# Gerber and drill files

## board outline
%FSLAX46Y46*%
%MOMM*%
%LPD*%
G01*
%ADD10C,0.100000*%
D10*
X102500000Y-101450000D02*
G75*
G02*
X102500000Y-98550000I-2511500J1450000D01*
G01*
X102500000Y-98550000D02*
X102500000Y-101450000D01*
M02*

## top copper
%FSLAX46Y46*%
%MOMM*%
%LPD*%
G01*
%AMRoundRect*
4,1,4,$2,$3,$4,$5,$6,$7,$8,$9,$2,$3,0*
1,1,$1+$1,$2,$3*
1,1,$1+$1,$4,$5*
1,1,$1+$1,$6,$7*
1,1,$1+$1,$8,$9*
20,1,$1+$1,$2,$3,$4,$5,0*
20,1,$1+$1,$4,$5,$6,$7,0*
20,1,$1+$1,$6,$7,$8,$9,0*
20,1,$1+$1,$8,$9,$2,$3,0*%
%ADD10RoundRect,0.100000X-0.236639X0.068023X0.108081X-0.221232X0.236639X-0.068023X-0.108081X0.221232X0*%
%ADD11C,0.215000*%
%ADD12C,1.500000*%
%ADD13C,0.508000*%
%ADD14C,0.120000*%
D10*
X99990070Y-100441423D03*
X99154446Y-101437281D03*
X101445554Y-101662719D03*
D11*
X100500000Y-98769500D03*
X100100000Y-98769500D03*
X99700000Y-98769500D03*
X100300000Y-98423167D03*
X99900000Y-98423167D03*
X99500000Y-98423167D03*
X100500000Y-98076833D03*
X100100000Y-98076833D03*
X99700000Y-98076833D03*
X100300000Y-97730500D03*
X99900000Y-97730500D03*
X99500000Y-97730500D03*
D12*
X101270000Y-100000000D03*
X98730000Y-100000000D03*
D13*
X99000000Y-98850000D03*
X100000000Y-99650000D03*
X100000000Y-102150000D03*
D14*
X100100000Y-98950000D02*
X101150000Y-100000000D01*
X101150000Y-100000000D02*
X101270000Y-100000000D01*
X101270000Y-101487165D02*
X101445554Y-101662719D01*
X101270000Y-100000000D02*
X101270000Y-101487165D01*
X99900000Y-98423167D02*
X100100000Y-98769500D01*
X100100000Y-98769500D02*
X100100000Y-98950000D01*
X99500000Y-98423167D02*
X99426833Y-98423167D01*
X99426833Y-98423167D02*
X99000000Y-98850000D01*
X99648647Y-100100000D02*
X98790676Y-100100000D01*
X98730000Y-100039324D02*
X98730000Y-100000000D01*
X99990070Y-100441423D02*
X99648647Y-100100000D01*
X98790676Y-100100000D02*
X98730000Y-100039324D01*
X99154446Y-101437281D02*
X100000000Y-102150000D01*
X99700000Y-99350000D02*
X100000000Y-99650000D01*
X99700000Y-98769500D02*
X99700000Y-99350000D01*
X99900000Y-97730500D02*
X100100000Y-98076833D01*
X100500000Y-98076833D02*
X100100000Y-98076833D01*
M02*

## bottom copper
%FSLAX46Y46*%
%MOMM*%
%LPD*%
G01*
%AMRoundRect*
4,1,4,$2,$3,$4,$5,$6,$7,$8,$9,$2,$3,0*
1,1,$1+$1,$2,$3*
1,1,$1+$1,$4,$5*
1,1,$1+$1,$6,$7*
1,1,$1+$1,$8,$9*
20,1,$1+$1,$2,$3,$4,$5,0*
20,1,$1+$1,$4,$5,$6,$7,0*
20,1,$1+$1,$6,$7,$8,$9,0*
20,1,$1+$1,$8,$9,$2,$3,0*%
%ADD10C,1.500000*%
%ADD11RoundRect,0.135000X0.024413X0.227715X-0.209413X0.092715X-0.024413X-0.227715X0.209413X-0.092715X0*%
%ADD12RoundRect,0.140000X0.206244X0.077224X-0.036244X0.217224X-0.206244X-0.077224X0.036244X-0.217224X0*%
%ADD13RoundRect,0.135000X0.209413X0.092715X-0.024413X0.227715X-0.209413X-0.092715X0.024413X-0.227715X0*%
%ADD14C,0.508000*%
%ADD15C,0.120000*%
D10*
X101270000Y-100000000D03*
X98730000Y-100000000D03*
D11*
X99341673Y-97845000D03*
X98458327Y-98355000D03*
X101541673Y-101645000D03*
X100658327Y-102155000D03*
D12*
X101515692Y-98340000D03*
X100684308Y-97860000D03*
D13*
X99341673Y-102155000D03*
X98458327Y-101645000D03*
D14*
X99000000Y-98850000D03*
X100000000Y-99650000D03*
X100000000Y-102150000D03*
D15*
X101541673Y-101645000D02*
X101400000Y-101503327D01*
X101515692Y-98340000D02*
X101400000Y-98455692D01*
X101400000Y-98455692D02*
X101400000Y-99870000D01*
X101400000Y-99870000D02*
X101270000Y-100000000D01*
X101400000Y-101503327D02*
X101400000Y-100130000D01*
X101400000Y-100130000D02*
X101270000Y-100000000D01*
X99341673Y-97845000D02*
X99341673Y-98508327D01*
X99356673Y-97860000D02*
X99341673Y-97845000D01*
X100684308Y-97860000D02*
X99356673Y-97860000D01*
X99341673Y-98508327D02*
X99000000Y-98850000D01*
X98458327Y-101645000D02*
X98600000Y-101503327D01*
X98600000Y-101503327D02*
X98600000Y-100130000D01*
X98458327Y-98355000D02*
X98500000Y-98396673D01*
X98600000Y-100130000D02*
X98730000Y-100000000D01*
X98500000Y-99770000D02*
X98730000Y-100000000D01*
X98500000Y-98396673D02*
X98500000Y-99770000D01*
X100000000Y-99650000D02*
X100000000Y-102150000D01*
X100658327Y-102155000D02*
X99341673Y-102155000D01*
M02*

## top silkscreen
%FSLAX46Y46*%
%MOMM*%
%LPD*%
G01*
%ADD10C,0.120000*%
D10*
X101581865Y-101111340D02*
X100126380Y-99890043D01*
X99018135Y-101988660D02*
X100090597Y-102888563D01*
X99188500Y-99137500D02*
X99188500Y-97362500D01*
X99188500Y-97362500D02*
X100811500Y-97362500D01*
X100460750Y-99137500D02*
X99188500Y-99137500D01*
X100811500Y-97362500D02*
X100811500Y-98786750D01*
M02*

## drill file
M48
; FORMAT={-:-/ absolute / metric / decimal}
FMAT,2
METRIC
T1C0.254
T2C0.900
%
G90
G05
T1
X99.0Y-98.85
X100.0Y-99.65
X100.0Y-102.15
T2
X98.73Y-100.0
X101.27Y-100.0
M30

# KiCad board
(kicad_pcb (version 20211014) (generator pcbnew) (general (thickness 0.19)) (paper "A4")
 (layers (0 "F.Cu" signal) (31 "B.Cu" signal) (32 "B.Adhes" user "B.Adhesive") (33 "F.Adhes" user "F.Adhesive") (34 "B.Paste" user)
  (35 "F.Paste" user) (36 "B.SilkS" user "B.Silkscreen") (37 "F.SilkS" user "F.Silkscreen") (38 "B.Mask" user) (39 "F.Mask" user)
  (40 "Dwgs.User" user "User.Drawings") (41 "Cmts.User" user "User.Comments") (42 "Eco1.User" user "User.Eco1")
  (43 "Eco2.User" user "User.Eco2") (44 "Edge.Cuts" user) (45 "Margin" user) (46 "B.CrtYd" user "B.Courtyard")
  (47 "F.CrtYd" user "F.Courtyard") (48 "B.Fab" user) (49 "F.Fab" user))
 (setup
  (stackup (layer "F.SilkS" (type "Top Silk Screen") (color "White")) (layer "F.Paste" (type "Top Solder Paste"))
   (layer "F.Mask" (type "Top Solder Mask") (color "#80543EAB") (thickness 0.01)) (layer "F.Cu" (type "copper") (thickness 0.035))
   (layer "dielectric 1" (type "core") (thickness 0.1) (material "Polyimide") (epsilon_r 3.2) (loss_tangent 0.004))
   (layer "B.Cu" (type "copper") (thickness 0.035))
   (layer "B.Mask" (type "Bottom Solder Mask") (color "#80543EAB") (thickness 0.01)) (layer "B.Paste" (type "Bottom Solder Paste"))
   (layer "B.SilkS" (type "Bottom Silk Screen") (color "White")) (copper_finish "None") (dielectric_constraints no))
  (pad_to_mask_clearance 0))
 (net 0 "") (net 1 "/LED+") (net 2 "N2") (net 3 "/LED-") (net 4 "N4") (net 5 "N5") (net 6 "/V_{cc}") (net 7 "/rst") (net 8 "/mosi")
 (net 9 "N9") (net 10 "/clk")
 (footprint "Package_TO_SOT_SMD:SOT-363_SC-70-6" (layer "F.Cu") (at 100.3 101.55 -40)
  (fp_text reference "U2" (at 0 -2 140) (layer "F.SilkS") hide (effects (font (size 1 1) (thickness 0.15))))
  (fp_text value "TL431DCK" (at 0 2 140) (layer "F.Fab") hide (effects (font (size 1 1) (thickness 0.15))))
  (fp_line (start 0.7 -1.16) (end -1.2 -1.16) (layer "F.SilkS") (width 0.12))
  (fp_line (start -0.7 1.16) (end 0.7 1.16) (layer "F.SilkS") (width 0.12))
  (pad "1" smd roundrect (at -0.95 -0.65 320) (size 0.65 0.4) (layers "F.Cu" "F.Paste" "F.Mask") (roundrect_rratio 0.25) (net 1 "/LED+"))
  (pad "3" smd roundrect (at -0.95 0.65 320) (size 0.65 0.4) (layers "F.Cu" "F.Paste" "F.Mask") (roundrect_rratio 0.25) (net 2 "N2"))
  (pad "6" smd roundrect (at 0.95 -0.65 320) (size 0.65 0.4) (layers "F.Cu" "F.Paste" "F.Mask") (roundrect_rratio 0.25) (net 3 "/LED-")))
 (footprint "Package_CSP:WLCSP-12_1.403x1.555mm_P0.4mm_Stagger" (layer "F.Cu") (at 100 98.25 180) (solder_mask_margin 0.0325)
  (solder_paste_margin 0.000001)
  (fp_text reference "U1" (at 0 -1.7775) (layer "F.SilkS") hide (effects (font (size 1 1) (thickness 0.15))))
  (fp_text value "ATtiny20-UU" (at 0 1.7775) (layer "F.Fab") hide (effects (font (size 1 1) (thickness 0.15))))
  (fp_line (start 0.8115 -0.8875) (end 0.8115 0.8875) (layer "F.SilkS") (width 0.12))
  (fp_line (start 0.8115 0.8875) (end -0.8115 0.8875) (layer "F.SilkS") (width 0.12))
  (fp_line (start -0.46075 -0.8875) (end 0.8115 -0.8875) (layer "F.SilkS") (width 0.12))
  (fp_line (start -0.8115 0.8875) (end -0.8115 -0.53675) (layer "F.SilkS") (width 0.12))
  (pad "A1" smd circle locked (at -0.5 -0.5195 180) (size 0.215 0.215) (layers "F.Cu" "F.Paste" "F.Mask") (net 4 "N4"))
  (pad "A3" smd circle locked (at -0.1 -0.5195 180) (size 0.215 0.215) (layers "F.Cu" "F.Paste" "F.Mask") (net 3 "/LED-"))
  (pad "A5" smd circle locked (at 0.3 -0.5195 180) (size 0.215 0.215) (layers "F.Cu" "F.Paste" "F.Mask") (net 2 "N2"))
  (pad "B2" smd circle locked (at -0.3 -0.173167 180) (size 0.215 0.215) (layers "F.Cu" "F.Paste" "F.Mask") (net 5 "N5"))
  (pad "B4" smd circle locked (at 0.1 -0.173167 180) (size 0.215 0.215) (layers "F.Cu" "F.Paste" "F.Mask") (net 3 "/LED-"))
  (pad "B6" smd circle locked (at 0.5 -0.173167 180) (size 0.215 0.215) (layers "F.Cu" "F.Paste" "F.Mask") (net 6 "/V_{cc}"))
  (pad "C1" smd circle locked (at -0.5 0.173167 180) (size 0.215 0.215) (layers "F.Cu" "F.Paste" "F.Mask") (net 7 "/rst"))
  (pad "C3" smd circle locked (at -0.1 0.173167 180) (size 0.215 0.215) (layers "F.Cu" "F.Paste" "F.Mask") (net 7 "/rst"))
  (pad "C5" smd circle locked (at 0.3 0.173167 180) (size 0.215 0.215) (layers "F.Cu" "F.Paste" "F.Mask") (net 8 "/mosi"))
  (pad "D2" smd circle locked (at -0.3 0.5195 180) (size 0.215 0.215) (layers "F.Cu" "F.Paste" "F.Mask") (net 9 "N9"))
  (pad "D4" smd circle locked (at 0.1 0.5195 180) (size 0.215 0.215) (layers "F.Cu" "F.Paste" "F.Mask") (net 7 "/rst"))
  (pad "D6" smd circle locked (at 0.5 0.5195 180) (size 0.215 0.215) (layers "F.Cu" "F.Paste" "F.Mask") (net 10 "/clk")))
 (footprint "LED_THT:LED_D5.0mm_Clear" (layer "B.Cu") (at 100 100 180)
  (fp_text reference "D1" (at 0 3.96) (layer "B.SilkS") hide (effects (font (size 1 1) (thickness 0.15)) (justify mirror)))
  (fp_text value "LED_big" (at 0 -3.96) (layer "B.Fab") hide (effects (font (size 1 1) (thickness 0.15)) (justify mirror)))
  (pad "1" thru_hole circle (at -1.27 0 180) (size 1.5 1.5) (drill 0.9) (layers *.Cu *.Mask) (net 3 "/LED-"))
  (pad "2" thru_hole circle (at 1.27 0 180) (size 1.5 1.5) (drill 0.9) (layers *.Cu *.Mask) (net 1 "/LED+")))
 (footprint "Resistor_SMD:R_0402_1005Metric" (layer "B.Cu") (at 98.9 98.1 -150)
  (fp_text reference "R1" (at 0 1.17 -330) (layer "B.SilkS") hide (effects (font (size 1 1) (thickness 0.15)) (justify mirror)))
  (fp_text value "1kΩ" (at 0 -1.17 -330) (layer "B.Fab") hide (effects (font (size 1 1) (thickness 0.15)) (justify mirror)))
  (pad "1" smd roundrect locked (at -0.51 0 210) (size 0.54 0.64) (layers "B.Cu" "B.Paste" "B.Mask") (roundrect_rratio 0.25)
   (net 6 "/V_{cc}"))
  (pad "2" smd roundrect locked (at 0.51 0 210) (size 0.54 0.64) (layers "B.Cu" "B.Paste" "B.Mask") (roundrect_rratio 0.25) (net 1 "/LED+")))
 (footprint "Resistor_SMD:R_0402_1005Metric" (layer "B.Cu") (at 101.1 101.9 -150)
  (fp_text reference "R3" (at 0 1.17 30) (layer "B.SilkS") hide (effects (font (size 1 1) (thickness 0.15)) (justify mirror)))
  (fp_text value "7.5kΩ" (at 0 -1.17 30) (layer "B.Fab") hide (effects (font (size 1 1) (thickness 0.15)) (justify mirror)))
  (pad "1" smd roundrect locked (at -0.51 0 210) (size 0.54 0.64) (layers "B.Cu" "B.Paste" "B.Mask") (roundrect_rratio 0.25) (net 3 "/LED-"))
  (pad "2" smd roundrect locked (at 0.51 0 210) (size 0.54 0.64) (layers "B.Cu" "B.Paste" "B.Mask") (roundrect_rratio 0.25) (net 2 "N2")))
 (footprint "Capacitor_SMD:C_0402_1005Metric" (layer "B.Cu") (at 101.1 98.1 150)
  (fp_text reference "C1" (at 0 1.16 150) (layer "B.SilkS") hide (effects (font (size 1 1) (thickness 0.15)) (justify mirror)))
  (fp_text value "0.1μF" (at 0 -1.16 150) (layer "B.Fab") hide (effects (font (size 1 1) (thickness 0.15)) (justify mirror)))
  (pad "1" smd roundrect locked (at -0.48 0 150) (size 0.56 0.62) (layers "B.Cu" "B.Paste" "B.Mask") (roundrect_rratio 0.25) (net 3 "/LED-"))
  (pad "2" smd roundrect locked (at 0.48 0 150) (size 0.56 0.62) (layers "B.Cu" "B.Paste" "B.Mask") (roundrect_rratio 0.25)
   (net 6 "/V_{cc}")))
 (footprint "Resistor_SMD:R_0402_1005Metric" (layer "B.Cu") (at 98.9 101.9 150)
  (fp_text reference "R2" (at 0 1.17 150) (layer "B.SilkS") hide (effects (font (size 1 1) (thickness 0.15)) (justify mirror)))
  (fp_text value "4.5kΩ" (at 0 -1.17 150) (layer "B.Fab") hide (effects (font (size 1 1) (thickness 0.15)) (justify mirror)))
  (pad "1" smd roundrect locked (at -0.51 0 150) (size 0.54 0.64) (layers "B.Cu" "B.Paste" "B.Mask") (roundrect_rratio 0.25) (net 2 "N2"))
  (pad "2" smd roundrect locked (at 0.51 0 150) (size 0.54 0.64) (layers "B.Cu" "B.Paste" "B.Mask") (roundrect_rratio 0.25) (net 1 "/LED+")))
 (gr_arc (start 102.5 101.45) (mid 97.088526 100) (end 102.5 98.55) (layer "Edge.Cuts") (width 0.1))
 (gr_line (start 102.5 98.55) (end 102.5 101.45) (layer "Edge.Cuts") (width 0.1))
 (segment (start 100.1 98.95) (end 101.15 100) (width 0.12) (layer "F.Cu") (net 3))
 (segment (start 101.15 100) (end 101.27 100) (width 0.12) (layer "F.Cu") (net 3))
 (segment (start 101.27 101.487165) (end 101.445554 101.662719) (width 0.12) (layer "F.Cu") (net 3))
 (segment (start 101.27 100) (end 101.27 101.487165) (width 0.12) (layer "F.Cu") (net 3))
 (segment (start 99.9 98.423167) (end 100.1 98.7695) (width 0.12) (layer "F.Cu") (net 3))
 (segment (start 100.1 98.7695) (end 100.1 98.95) (width 0.12) (layer "F.Cu") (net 3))
 (segment (start 101.541673 101.645) (end 101.4 101.503327) (width 0.12) (layer "B.Cu") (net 3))
 (segment (start 101.515692 98.34) (end 101.4 98.455692) (width 0.12) (layer "B.Cu") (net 3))
 (segment (start 101.4 98.455692) (end 101.4 99.87) (width 0.12) (layer "B.Cu") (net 3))
 (segment (start 101.4 99.87) (end 101.27 100) (width 0.12) (layer "B.Cu") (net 3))
 (segment (start 101.4 101.503327) (end 101.4 100.13) (width 0.12) (layer "B.Cu") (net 3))
 (segment (start 101.4 100.13) (end 101.27 100) (width 0.12) (layer "B.Cu") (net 3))
 (segment (start 99.5 98.423167) (end 99.426833 98.423167) (width 0.12) (layer "F.Cu") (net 6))
 (segment (start 99.426833 98.423167) (end 99 98.85) (width 0.12) (layer "F.Cu") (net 6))
 (via (at 99 98.85) (size 0.508) (drill 0.254) (layers "F.Cu" "B.Cu") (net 6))
 (segment (start 99.341673 97.845) (end 99.341673 98.508327) (width 0.12) (layer "B.Cu") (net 6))
 (segment (start 99.356673 97.86) (end 99.341673 97.845) (width 0.12) (layer "B.Cu") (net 6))
 (segment (start 100.684308 97.86) (end 99.356673 97.86) (width 0.12) (layer "B.Cu") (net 6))
 (segment (start 99.341673 98.508327) (end 99 98.85) (width 0.12) (layer "B.Cu") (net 6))
 (segment (start 99.648647 100.1) (end 98.790676 100.1) (width 0.12) (layer "F.Cu") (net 1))
 (segment (start 98.73 100.039324) (end 98.73 100) (width 0.12) (layer "F.Cu") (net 1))
 (segment (start 99.99007 100.441423) (end 99.648647 100.1) (width 0.12) (layer "F.Cu") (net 1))
 (segment (start 98.790676 100.1) (end 98.73 100.039324) (width 0.12) (layer "F.Cu") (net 1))
 (segment (start 98.458327 101.645) (end 98.6 101.503327) (width 0.12) (layer "B.Cu") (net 1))
 (segment (start 98.6 101.503327) (end 98.6 100.13) (width 0.12) (layer "B.Cu") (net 1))
 (segment (start 98.458327 98.355) (end 98.5 98.396673) (width 0.12) (layer "B.Cu") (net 1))
 (segment (start 98.6 100.13) (end 98.73 100) (width 0.12) (layer "B.Cu") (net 1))
 (segment (start 98.5 99.77) (end 98.73 100) (width 0.12) (layer "B.Cu") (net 1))
 (segment (start 98.5 98.396673) (end 98.5 99.77) (width 0.12) (layer "B.Cu") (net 1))
 (segment (start 99.154446 101.437281) (end 100 102.15) (width 0.12) (layer "F.Cu") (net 2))
 (segment (start 99.7 99.35) (end 100 99.65) (width 0.12) (layer "F.Cu") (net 2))
 (segment (start 99.7 98.7695) (end 99.7 99.35) (width 0.12) (layer "F.Cu") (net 2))
 (via (at 100 99.65) (size 0.508) (drill 0.254) (layers "F.Cu" "B.Cu") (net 2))
 (via (at 100 102.15) (size 0.508) (drill 0.254) (layers "F.Cu" "B.Cu") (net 2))
 (segment (start 100 99.65) (end 100 102.15) (width 0.12) (layer "B.Cu") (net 2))
 (segment (start 100.658327 102.155) (end 99.341673 102.155) (width 0.12) (layer "B.Cu") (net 2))
 (segment (start 99.9 97.7305) (end 100.1 98.076833) (width 0.12) (layer "F.Cu") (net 7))
 (segment (start 100.5 98.076833) (end 100.1 98.076833) (width 0.12) (layer "F.Cu") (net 7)))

